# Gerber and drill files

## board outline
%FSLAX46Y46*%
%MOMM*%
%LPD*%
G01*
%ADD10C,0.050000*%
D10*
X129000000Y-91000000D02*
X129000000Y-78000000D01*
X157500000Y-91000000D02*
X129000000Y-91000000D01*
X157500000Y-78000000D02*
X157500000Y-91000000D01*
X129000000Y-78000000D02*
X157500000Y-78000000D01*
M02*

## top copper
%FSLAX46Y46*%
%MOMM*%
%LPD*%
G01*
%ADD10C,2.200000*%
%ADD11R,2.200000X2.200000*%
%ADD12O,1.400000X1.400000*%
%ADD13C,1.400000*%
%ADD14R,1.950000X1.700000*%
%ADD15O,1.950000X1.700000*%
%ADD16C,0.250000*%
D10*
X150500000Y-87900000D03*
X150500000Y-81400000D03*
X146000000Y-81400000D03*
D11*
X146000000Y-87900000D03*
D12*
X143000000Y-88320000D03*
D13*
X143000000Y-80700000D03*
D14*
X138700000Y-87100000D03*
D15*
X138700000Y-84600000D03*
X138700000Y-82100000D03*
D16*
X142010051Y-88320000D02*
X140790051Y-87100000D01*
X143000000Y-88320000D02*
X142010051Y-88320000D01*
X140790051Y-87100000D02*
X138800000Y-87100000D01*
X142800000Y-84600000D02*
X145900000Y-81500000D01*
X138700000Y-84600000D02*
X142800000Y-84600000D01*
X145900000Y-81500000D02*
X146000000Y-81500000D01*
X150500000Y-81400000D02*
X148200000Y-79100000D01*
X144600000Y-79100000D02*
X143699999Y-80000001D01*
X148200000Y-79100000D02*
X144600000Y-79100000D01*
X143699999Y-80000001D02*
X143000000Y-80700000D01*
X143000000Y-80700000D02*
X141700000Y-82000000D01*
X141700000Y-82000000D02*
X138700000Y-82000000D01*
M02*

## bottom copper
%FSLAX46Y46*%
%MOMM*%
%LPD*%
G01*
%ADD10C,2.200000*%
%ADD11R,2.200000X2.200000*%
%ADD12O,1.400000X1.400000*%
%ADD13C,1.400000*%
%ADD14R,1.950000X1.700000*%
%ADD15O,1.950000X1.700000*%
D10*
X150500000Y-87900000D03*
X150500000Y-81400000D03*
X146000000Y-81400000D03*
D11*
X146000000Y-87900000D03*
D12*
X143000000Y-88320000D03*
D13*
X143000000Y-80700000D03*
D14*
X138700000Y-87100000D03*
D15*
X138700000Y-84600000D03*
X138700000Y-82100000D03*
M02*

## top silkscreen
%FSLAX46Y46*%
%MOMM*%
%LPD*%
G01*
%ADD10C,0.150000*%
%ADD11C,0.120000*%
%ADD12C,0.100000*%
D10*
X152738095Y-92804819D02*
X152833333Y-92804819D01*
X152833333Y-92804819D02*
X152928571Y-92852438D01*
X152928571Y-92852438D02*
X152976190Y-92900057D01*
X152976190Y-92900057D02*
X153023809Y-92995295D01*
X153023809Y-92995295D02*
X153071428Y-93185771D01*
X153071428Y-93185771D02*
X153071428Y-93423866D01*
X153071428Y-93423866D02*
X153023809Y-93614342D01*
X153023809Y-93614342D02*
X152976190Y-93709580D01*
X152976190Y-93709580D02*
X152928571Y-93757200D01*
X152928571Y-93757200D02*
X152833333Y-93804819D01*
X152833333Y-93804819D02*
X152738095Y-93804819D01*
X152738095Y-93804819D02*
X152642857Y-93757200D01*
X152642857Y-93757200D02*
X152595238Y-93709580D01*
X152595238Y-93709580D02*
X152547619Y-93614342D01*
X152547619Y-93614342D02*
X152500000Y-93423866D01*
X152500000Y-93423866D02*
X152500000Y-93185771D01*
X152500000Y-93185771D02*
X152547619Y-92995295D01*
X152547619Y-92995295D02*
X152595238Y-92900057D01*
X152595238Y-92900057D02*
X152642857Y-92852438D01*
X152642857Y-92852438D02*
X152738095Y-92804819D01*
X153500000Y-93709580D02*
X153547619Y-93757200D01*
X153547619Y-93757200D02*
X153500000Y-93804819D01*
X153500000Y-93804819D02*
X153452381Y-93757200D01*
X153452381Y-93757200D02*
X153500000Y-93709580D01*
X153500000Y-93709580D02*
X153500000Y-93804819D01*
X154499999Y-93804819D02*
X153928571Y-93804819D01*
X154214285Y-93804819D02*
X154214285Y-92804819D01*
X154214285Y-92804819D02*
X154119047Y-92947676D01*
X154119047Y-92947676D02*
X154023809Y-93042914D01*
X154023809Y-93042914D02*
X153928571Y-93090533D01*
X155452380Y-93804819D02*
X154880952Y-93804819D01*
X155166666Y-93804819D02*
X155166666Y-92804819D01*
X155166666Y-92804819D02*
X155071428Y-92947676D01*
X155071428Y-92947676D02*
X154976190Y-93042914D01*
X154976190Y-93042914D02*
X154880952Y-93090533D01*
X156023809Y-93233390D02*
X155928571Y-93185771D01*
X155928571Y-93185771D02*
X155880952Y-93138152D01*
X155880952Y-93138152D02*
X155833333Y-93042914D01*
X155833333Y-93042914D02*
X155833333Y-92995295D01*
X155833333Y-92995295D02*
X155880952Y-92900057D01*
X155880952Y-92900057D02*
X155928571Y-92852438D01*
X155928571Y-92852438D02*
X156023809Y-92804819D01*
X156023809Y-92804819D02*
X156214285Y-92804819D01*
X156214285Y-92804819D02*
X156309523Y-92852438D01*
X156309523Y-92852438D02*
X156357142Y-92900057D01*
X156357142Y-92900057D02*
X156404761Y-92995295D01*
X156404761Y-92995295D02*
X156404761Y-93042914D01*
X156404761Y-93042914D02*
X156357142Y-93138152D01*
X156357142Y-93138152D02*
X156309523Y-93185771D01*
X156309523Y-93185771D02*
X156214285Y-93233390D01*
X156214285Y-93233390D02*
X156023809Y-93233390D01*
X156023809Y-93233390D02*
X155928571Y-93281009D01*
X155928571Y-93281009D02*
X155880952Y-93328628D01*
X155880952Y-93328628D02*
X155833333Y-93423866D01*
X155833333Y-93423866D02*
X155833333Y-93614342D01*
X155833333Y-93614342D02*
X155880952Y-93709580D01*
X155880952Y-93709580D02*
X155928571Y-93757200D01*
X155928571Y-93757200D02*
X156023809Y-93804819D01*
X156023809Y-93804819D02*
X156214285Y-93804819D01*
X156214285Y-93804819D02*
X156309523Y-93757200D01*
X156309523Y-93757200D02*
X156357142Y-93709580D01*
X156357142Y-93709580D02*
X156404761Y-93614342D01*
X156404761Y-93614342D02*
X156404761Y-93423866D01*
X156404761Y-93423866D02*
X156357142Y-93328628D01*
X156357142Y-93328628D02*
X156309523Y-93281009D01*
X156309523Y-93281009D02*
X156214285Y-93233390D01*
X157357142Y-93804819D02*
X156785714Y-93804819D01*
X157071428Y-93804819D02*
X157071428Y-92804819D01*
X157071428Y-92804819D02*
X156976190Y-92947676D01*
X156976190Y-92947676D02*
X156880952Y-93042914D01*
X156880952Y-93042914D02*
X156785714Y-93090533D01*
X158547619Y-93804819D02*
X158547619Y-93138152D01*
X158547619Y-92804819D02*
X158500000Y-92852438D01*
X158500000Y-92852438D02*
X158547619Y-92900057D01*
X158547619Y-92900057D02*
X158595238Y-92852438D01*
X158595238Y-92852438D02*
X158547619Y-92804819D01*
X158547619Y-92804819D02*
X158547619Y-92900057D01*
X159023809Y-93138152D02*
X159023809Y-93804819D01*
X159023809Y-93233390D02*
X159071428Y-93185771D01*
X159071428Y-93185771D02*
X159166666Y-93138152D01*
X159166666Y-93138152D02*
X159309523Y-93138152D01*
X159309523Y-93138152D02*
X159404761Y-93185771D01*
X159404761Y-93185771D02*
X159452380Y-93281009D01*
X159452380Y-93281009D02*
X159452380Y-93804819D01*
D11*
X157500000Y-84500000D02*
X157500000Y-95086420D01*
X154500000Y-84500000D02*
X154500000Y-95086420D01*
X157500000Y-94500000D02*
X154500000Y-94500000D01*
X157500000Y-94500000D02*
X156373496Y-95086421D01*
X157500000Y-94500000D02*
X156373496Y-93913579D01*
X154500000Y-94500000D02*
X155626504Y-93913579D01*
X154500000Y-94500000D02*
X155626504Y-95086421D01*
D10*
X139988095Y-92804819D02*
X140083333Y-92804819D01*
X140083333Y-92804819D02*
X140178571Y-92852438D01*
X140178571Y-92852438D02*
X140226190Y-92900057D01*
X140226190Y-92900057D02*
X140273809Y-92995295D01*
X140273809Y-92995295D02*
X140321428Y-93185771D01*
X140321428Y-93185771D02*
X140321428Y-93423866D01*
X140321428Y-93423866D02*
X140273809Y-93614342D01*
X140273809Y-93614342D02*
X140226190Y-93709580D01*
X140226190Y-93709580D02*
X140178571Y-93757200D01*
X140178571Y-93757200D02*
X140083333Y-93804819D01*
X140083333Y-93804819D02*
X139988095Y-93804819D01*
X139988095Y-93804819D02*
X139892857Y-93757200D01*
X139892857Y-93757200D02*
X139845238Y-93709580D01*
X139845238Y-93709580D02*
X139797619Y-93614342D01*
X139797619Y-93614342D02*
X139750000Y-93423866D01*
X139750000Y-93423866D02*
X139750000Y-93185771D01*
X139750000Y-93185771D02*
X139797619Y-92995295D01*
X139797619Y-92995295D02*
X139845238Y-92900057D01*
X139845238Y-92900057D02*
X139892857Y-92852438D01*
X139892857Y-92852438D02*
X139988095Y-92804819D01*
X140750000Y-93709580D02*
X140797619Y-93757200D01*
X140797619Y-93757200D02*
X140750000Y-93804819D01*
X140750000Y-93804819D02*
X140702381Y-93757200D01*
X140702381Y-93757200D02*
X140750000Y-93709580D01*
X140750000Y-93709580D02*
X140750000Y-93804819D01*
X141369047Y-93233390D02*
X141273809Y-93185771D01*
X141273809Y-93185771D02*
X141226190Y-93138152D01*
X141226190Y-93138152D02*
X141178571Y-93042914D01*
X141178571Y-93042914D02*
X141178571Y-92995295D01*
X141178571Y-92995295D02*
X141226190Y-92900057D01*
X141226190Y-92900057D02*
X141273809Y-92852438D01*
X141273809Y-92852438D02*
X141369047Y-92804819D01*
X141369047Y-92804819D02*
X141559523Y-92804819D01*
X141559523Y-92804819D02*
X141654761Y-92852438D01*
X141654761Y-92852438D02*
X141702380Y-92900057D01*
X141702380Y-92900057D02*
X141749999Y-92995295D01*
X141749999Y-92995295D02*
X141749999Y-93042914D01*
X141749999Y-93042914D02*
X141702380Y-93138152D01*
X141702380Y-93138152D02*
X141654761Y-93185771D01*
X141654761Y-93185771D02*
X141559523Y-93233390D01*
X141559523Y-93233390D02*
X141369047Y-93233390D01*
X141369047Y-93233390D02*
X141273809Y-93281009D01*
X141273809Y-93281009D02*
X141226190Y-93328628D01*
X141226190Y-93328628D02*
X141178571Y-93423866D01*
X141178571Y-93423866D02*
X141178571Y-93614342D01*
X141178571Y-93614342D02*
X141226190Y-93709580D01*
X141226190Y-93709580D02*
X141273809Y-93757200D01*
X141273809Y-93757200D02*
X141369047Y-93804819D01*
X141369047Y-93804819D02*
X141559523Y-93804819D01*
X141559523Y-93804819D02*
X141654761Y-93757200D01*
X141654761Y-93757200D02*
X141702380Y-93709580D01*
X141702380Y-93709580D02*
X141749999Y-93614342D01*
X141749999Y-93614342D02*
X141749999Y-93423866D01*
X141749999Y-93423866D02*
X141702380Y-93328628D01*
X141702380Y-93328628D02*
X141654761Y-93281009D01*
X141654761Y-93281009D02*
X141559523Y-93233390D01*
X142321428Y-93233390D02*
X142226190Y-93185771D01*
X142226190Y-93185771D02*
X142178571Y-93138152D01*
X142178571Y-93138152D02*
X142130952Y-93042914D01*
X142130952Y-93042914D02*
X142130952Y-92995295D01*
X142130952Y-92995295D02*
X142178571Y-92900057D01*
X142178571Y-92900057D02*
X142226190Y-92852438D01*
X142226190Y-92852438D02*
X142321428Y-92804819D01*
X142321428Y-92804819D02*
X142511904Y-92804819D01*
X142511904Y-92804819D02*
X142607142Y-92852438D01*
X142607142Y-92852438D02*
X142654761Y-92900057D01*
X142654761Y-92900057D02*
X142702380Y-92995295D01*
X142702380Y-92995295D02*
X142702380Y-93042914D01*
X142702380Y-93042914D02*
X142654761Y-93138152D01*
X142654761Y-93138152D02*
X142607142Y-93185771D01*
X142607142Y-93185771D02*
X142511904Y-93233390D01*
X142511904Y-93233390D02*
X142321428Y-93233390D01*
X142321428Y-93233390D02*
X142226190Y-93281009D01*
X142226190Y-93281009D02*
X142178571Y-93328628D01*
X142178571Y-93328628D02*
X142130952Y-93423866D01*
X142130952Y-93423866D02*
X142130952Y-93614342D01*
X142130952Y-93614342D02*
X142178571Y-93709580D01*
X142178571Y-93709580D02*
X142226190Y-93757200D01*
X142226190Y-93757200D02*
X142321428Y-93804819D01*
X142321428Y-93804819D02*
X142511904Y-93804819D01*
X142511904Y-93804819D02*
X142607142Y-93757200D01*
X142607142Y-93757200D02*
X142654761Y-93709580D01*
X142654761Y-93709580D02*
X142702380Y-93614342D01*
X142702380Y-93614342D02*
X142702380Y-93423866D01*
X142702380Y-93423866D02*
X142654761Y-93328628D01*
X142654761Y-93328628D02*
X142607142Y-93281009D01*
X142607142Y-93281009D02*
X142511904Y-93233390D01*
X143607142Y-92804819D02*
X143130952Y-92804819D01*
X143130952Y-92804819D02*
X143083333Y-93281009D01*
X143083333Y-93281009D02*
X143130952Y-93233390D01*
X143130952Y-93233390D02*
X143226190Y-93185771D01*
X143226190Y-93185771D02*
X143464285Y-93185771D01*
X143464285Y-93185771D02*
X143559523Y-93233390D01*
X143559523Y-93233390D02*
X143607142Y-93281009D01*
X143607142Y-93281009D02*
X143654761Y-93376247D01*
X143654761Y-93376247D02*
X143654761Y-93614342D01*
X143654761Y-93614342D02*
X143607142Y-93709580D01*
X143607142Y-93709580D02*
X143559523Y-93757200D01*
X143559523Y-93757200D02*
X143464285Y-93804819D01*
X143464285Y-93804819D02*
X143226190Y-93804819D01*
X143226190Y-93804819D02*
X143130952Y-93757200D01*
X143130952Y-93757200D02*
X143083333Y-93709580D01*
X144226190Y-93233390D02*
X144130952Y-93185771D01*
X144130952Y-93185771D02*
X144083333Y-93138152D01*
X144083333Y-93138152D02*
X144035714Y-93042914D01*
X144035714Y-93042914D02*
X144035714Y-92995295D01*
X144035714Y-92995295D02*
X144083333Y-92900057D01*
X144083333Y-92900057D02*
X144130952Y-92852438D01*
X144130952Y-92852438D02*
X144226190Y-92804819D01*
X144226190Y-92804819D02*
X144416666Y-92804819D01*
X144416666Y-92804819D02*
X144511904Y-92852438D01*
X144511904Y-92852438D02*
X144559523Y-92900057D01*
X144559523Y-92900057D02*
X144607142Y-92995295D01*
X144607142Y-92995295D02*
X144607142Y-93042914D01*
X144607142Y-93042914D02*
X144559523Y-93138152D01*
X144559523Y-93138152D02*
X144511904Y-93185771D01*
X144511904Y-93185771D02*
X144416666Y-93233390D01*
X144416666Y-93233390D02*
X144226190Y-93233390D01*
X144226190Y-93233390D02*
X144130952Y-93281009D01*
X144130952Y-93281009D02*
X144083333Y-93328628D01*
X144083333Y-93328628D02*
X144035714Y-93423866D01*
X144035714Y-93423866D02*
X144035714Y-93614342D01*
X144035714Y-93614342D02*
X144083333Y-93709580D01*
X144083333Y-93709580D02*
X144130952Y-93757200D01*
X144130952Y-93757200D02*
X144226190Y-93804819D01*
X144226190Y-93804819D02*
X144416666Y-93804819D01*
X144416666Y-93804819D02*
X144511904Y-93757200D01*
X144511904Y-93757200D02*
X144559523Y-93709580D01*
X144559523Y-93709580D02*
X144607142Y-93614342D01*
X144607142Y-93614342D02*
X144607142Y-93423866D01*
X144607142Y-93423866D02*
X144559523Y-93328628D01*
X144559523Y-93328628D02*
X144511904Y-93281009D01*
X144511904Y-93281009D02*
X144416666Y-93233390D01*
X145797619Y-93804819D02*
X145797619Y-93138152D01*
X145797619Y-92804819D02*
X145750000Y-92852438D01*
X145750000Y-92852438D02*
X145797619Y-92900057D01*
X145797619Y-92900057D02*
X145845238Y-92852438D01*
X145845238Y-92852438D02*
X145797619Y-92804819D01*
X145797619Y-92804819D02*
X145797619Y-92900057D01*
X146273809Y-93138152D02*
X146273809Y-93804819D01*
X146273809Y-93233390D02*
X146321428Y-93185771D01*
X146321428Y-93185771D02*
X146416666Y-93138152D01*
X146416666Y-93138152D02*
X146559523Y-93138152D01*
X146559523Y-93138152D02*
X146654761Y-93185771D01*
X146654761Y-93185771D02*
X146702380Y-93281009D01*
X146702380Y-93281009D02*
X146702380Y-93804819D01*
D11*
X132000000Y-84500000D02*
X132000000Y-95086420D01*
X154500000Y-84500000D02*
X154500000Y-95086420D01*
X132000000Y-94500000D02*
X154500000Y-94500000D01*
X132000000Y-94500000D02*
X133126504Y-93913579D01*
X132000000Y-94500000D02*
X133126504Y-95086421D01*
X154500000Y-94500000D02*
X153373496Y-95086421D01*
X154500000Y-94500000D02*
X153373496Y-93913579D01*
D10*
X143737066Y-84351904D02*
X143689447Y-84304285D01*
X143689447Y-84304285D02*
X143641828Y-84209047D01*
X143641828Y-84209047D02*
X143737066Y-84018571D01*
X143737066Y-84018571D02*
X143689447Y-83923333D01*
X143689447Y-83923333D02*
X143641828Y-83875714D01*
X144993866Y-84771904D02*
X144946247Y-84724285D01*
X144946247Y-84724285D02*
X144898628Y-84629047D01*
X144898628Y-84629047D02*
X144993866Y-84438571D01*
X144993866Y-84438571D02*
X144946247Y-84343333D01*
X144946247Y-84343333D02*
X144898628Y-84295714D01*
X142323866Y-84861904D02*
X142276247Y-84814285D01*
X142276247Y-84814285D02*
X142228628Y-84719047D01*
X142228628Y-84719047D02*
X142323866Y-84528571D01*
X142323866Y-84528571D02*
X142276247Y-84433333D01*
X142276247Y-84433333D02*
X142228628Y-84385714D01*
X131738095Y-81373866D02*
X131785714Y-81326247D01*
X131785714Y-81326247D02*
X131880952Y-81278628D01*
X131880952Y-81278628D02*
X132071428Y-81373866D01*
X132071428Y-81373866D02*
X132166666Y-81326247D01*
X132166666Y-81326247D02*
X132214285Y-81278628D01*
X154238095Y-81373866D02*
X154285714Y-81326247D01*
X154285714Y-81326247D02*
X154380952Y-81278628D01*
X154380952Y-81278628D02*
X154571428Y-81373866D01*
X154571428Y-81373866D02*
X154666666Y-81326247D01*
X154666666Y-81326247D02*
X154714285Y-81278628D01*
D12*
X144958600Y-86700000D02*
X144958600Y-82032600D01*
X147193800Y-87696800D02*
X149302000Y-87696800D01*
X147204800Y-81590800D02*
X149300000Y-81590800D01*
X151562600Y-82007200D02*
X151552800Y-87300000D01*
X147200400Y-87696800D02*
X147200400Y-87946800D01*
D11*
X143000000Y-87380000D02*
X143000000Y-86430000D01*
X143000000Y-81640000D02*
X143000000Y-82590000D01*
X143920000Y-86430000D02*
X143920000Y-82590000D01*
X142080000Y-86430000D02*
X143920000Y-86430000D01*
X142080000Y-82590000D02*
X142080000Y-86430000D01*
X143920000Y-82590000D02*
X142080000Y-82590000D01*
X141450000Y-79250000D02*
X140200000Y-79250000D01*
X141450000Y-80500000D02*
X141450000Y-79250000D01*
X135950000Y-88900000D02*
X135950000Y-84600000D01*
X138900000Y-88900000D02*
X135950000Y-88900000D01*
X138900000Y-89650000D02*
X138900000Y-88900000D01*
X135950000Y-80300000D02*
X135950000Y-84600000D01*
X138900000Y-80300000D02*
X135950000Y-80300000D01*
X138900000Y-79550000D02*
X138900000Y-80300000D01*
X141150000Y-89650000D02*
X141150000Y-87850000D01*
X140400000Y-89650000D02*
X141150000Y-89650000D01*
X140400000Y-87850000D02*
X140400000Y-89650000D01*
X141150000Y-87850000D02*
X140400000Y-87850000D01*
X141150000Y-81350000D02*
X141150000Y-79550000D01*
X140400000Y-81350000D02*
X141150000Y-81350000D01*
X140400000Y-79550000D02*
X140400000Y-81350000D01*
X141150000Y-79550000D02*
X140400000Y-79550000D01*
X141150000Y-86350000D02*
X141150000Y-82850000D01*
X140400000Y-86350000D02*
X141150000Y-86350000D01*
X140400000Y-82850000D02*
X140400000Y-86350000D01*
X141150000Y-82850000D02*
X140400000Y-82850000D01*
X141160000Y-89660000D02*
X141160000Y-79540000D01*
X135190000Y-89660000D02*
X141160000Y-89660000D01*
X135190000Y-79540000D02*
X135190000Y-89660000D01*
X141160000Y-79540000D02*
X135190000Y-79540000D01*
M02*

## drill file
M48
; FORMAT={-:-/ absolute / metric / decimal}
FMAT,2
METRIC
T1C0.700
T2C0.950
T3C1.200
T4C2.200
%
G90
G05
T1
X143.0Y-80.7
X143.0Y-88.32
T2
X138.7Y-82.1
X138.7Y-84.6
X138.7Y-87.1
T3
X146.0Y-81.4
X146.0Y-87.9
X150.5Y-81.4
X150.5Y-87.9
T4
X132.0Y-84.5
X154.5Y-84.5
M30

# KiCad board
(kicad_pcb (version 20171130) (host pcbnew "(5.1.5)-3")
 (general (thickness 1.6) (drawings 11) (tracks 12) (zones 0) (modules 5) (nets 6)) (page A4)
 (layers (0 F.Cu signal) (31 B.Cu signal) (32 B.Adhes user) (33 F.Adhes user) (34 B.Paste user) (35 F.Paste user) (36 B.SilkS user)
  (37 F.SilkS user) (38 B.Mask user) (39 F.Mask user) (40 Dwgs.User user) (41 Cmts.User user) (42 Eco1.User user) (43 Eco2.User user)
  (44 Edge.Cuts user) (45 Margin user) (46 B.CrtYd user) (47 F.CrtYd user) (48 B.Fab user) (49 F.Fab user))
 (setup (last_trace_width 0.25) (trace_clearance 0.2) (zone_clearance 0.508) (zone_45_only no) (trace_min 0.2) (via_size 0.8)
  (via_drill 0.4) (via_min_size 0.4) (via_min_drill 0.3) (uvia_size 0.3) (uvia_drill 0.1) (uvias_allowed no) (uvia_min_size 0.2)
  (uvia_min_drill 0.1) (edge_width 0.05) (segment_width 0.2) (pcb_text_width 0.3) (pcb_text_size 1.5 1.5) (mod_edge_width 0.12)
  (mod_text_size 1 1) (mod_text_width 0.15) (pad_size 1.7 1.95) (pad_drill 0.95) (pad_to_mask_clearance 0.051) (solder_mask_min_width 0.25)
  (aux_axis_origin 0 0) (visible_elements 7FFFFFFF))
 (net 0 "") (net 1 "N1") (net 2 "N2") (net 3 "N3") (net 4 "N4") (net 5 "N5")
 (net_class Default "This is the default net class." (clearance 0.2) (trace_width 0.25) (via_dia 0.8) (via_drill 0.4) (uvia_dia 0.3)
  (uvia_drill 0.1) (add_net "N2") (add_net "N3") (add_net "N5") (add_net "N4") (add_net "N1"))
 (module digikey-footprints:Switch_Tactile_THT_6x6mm (layer F.Cu) (at 146 87.9 90)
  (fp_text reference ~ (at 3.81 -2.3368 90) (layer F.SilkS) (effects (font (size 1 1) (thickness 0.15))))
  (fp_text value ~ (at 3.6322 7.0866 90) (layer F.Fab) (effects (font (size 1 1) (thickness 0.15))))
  (fp_line (start 1.2 -1.0414) (end 5.8674 -1.0414) (layer F.SilkS) (width 0.1))
  (fp_line (start 0.2032 1.1938) (end 0.2032 3.302) (layer F.SilkS) (width 0.1))
  (fp_line (start 6.3092 1.2048) (end 6.3092 3.3) (layer F.SilkS) (width 0.1))
  (fp_line (start 5.8928 5.5626) (end 0.6 5.5528) (layer F.SilkS) (width 0.1))
  (fp_line (start 0.2032 1.2004) (end -0.0468 1.2004) (layer F.SilkS) (width 0.1))
  (pad 3 thru_hole circle (at 0 4.5 90) (size 2.2 2.2) (drill 1.2) (layers *.Cu *.Mask) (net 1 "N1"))
  (pad 4 thru_hole circle (at 6.5 4.5 90) (size 2.2 2.2) (drill 1.2) (layers *.Cu *.Mask) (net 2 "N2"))
  (pad 2 thru_hole circle (at 6.5 0 90) (size 2.2 2.2) (drill 1.2) (layers *.Cu *.Mask) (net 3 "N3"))
  (pad 1 thru_hole rect (at 0 0 90) (size 2.2 2.2) (drill 1.2) (layers *.Cu *.Mask) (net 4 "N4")))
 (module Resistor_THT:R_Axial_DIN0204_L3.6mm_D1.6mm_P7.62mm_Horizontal (layer F.Cu) (at 143 80.7 270)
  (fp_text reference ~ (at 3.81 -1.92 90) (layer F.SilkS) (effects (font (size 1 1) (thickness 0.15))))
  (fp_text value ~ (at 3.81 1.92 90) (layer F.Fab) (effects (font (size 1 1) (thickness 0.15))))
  (fp_line (start 6.68 0) (end 5.73 0) (layer F.SilkS) (width 0.12))
  (fp_line (start 0.94 0) (end 1.89 0) (layer F.SilkS) (width 0.12))
  (fp_line (start 5.73 -0.92) (end 1.89 -0.92) (layer F.SilkS) (width 0.12))
  (fp_line (start 5.73 0.92) (end 5.73 -0.92) (layer F.SilkS) (width 0.12))
  (fp_line (start 1.89 0.92) (end 5.73 0.92) (layer F.SilkS) (width 0.12))
  (fp_line (start 1.89 -0.92) (end 1.89 0.92) (layer F.SilkS) (width 0.12))
  (pad 2 thru_hole oval (at 7.62 0 270) (size 1.4 1.4) (drill 0.7) (layers *.Cu *.Mask) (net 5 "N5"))
  (pad 1 thru_hole circle (at 0 0 270) (size 1.4 1.4) (drill 0.7) (layers *.Cu *.Mask) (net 2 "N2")))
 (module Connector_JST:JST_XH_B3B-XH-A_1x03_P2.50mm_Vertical (layer F.Cu) (at 138.7 82.1 270)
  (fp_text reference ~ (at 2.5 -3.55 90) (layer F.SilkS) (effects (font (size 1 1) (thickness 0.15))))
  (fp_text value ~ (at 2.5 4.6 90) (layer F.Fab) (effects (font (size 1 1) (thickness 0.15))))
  (fp_line (start -2.85 -2.75) (end -2.85 -1.5) (layer F.SilkS) (width 0.12))
  (fp_line (start -1.6 -2.75) (end -2.85 -2.75) (layer F.SilkS) (width 0.12))
  (fp_line (start 6.8 2.75) (end 2.5 2.75) (layer F.SilkS) (width 0.12))
  (fp_line (start 6.8 -0.2) (end 6.8 2.75) (layer F.SilkS) (width 0.12))
  (fp_line (start 7.55 -0.2) (end 6.8 -0.2) (layer F.SilkS) (width 0.12))
  (fp_line (start -1.8 2.75) (end 2.5 2.75) (layer F.SilkS) (width 0.12))
  (fp_line (start -1.8 -0.2) (end -1.8 2.75) (layer F.SilkS) (width 0.12))
  (fp_line (start -2.55 -0.2) (end -1.8 -0.2) (layer F.SilkS) (width 0.12))
  (fp_line (start 7.55 -2.45) (end 5.75 -2.45) (layer F.SilkS) (width 0.12))
  (fp_line (start 7.55 -1.7) (end 7.55 -2.45) (layer F.SilkS) (width 0.12))
  (fp_line (start 5.75 -1.7) (end 7.55 -1.7) (layer F.SilkS) (width 0.12))
  (fp_line (start 5.75 -2.45) (end 5.75 -1.7) (layer F.SilkS) (width 0.12))
  (fp_line (start -0.75 -2.45) (end -2.55 -2.45) (layer F.SilkS) (width 0.12))
  (fp_line (start -0.75 -1.7) (end -0.75 -2.45) (layer F.SilkS) (width 0.12))
  (fp_line (start -2.55 -1.7) (end -0.75 -1.7) (layer F.SilkS) (width 0.12))
  (fp_line (start -2.55 -2.45) (end -2.55 -1.7) (layer F.SilkS) (width 0.12))
  (fp_line (start 4.25 -2.45) (end 0.75 -2.45) (layer F.SilkS) (width 0.12))
  (fp_line (start 4.25 -1.7) (end 4.25 -2.45) (layer F.SilkS) (width 0.12))
  (fp_line (start 0.75 -1.7) (end 4.25 -1.7) (layer F.SilkS) (width 0.12))
  (fp_line (start 0.75 -2.45) (end 0.75 -1.7) (layer F.SilkS) (width 0.12))
  (fp_line (start 7.56 -2.46) (end -2.56 -2.46) (layer F.SilkS) (width 0.12))
  (fp_line (start 7.56 3.51) (end 7.56 -2.46) (layer F.SilkS) (width 0.12))
  (fp_line (start -2.56 3.51) (end 7.56 3.51) (layer F.SilkS) (width 0.12))
  (fp_line (start -2.56 -2.46) (end -2.56 3.51) (layer F.SilkS) (width 0.12))
  (pad GND thru_hole rect (at 5 0 270) (size 1.7 1.95) (drill 0.95) (layers *.Cu *.Mask) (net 5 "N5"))
  (pad VCC thru_hole oval (at 2.5 0 270) (size 1.7 1.95) (drill 0.95) (layers *.Cu *.Mask) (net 3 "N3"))
  (pad OUT thru_hole oval (at 0 0 270) (size 1.7 1.95) (drill 0.95) (layers *.Cu *.Mask) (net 2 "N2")))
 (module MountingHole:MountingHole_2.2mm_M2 (layer F.Cu) (at 132 84.5)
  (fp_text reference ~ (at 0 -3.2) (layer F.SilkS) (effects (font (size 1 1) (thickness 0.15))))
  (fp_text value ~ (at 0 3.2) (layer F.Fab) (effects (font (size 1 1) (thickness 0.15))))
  (pad 1 np_thru_hole circle (at 0 0) (size 2.2 2.2) (drill 2.2) (layers *.Cu *.Mask)))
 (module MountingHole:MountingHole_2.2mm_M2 (layer F.Cu) (at 154.5 84.5)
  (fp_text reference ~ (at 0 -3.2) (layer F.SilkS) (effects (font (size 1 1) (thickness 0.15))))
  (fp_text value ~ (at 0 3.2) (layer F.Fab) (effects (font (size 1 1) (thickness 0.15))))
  (pad 1 np_thru_hole circle (at 0 0) (size 2.2 2.2) (drill 2.2) (layers *.Cu *.Mask)))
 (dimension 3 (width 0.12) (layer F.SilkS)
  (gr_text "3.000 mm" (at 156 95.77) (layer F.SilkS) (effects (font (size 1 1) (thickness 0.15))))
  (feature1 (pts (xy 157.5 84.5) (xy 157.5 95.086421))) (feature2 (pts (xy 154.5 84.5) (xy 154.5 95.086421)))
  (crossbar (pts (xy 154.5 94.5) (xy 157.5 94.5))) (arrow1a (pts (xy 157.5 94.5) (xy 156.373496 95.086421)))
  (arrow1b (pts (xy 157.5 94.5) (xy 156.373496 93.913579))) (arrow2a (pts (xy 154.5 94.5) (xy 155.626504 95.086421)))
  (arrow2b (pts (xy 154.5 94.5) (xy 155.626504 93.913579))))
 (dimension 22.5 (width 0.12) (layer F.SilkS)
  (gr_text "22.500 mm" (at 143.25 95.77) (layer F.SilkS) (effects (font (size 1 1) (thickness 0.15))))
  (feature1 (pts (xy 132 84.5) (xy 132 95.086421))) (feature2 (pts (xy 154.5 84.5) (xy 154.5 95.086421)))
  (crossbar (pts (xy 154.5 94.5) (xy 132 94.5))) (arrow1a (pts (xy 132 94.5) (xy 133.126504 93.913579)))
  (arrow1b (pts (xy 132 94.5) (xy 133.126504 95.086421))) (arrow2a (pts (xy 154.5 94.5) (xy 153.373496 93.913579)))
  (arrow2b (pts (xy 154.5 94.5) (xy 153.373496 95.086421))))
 (gr_line (start 129 91) (end 129 78) (layer Edge.Cuts) (width 0.05))
 (gr_line (start 157.5 91) (end 129 91) (layer Edge.Cuts) (width 0.05))
 (gr_line (start 157.5 78) (end 157.5 91) (layer Edge.Cuts) (width 0.05))
 (gr_line (start 129 78) (end 157.5 78) (layer Edge.Cuts) (width 0.05))
 (segment (start 142.010051 88.32) (end 140.790051 87.1) (width 0.25) (layer F.Cu) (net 5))
 (segment (start 143 88.32) (end 142.010051 88.32) (width 0.25) (layer F.Cu) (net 5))
 (segment (start 140.790051 87.1) (end 138.8 87.1) (width 0.25) (layer F.Cu) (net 5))
 (segment (start 142.8 84.6) (end 145.9 81.5) (width 0.25) (layer F.Cu) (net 3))
 (segment (start 138.7 84.6) (end 142.8 84.6) (width 0.25) (layer F.Cu) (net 3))
 (segment (start 145.9 81.5) (end 146 81.5) (width 0.25) (layer F.Cu) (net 3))
 (segment (start 150.5 81.4) (end 148.2 79.1) (width 0.25) (layer F.Cu) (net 2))
 (segment (start 144.6 79.1) (end 143.699999 80.000001) (width 0.25) (layer F.Cu) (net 2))
 (segment (start 148.2 79.1) (end 144.6 79.1) (width 0.25) (layer F.Cu) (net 2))
 (segment (start 143.699999 80.000001) (end 143 80.7) (width 0.25) (layer F.Cu) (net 2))
 (segment (start 143 80.7) (end 141.7 82) (width 0.25) (layer F.Cu) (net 2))
 (segment (start 141.7 82) (end 138.7 82) (width 0.25) (layer F.Cu) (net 2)))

